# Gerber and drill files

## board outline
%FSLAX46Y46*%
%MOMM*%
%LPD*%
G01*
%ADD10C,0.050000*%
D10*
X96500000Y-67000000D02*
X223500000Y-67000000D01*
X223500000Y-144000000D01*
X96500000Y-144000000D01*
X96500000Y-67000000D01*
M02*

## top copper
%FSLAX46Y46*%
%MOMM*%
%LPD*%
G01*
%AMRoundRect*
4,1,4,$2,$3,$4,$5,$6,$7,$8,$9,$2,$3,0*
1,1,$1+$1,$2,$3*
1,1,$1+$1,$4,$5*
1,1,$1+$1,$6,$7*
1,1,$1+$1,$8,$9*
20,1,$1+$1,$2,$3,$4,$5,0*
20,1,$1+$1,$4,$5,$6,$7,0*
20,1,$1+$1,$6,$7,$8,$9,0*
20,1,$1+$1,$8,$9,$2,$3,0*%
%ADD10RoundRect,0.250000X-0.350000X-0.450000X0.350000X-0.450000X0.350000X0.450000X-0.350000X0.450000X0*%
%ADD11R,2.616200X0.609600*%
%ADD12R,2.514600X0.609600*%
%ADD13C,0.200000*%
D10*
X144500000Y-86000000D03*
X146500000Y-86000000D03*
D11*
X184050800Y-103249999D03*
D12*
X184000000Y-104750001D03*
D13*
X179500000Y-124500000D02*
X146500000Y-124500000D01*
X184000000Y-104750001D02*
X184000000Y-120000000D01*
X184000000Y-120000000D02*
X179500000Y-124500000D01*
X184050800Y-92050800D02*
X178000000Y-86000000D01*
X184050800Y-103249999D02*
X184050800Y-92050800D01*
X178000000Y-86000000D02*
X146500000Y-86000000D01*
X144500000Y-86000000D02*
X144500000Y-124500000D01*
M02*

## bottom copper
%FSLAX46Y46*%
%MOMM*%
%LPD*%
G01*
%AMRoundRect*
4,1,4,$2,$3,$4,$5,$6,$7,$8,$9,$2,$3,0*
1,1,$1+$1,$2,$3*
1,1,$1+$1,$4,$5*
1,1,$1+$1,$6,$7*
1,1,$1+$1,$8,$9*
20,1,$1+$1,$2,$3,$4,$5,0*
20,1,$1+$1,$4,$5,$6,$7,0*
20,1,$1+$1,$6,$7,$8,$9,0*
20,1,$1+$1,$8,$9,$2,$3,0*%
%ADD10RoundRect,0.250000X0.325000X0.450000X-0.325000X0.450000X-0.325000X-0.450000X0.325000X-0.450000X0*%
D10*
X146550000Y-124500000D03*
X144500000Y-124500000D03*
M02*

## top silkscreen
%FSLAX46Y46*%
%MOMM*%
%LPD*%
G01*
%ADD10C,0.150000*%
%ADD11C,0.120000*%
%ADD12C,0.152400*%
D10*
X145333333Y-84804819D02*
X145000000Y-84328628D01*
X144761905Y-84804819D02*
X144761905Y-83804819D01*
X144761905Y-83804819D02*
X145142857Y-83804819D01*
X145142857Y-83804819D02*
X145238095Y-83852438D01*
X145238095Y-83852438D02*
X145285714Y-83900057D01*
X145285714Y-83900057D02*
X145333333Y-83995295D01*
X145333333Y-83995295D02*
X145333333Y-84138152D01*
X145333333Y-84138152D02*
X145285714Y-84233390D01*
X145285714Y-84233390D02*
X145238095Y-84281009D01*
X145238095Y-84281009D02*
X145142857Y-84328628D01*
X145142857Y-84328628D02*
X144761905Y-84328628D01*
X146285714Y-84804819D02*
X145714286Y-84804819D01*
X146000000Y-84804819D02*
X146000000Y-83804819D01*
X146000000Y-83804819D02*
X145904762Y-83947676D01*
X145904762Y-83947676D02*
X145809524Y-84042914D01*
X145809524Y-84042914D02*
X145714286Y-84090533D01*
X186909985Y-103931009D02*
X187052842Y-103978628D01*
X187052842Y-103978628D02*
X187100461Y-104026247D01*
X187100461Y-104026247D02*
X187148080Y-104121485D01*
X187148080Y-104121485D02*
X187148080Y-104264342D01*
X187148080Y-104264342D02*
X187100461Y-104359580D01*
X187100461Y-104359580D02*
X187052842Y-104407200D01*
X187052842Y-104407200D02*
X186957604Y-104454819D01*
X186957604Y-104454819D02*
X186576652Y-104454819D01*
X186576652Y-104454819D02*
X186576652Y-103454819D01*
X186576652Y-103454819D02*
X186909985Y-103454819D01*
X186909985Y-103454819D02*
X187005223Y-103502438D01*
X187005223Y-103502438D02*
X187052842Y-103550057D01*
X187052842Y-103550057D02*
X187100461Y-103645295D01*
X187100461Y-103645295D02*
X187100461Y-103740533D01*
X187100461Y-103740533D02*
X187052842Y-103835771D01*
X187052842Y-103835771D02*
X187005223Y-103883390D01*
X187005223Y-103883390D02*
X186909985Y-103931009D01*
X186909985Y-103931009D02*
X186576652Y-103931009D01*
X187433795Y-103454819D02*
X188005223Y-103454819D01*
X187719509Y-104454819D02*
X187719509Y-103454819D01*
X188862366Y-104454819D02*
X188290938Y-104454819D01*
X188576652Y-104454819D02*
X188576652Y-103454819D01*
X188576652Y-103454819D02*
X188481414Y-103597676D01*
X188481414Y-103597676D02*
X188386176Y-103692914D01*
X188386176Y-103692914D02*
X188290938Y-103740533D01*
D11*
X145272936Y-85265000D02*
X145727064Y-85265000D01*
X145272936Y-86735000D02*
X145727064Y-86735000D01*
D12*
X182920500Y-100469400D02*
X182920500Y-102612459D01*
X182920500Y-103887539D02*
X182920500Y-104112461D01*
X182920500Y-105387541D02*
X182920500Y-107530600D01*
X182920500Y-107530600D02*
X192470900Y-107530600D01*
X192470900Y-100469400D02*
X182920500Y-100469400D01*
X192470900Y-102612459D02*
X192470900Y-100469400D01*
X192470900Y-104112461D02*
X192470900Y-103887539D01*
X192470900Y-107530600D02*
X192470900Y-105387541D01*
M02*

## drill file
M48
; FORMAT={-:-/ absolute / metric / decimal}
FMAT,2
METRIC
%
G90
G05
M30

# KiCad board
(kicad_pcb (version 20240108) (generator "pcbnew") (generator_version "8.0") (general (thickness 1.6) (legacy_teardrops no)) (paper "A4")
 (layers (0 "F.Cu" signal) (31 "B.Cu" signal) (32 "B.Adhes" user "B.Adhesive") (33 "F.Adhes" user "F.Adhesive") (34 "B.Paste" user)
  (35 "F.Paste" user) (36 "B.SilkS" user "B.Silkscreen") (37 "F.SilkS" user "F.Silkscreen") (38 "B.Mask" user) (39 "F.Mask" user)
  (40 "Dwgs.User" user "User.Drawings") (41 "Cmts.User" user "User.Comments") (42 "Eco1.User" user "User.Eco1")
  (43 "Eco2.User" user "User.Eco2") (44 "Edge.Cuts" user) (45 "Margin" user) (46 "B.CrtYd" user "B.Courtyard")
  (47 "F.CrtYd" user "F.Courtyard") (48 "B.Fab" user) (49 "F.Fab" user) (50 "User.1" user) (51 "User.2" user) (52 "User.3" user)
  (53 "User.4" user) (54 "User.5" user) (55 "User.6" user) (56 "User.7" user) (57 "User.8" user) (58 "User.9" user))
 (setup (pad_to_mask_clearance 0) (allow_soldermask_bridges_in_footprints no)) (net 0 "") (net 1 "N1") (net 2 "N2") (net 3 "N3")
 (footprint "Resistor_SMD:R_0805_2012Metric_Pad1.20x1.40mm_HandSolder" (layer "F.Cu") (at 145.5 86)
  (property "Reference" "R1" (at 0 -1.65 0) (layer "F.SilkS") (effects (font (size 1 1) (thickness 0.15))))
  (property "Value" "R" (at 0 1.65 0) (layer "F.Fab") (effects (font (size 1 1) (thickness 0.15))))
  (fp_line (start -0.227064 -0.735) (end 0.227064 -0.735) (stroke (width 0.12) (type solid)) (layer "F.SilkS"))
  (fp_line (start -0.227064 0.735) (end 0.227064 0.735) (stroke (width 0.12) (type solid)) (layer "F.SilkS"))
  (pad "1" smd roundrect (at -1 0) (size 1.2 1.4) (layers "F.Cu" "F.Paste" "F.Mask") (roundrect_rratio 0.208333) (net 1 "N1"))
  (pad "2" smd roundrect (at 1 0) (size 1.2 1.4) (layers "F.Cu" "F.Paste" "F.Mask") (roundrect_rratio 0.208333) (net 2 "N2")))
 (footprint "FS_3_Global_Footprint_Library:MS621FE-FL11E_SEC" (layer "F.Cu") (at 187.6957 104)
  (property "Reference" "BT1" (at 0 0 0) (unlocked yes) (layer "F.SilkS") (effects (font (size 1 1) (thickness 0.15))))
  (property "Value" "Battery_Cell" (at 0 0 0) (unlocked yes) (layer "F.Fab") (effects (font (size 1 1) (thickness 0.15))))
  (fp_line (start -4.7752 -3.5306) (end -4.7752 -1.387541) (stroke (width 0.1524) (type solid)) (layer "F.SilkS"))
  (fp_line (start -4.7752 -0.112461) (end -4.7752 0.112461) (stroke (width 0.1524) (type solid)) (layer "F.SilkS"))
  (fp_line (start -4.7752 1.387541) (end -4.7752 3.5306) (stroke (width 0.1524) (type solid)) (layer "F.SilkS"))
  (fp_line (start -4.7752 3.5306) (end 4.7752 3.5306) (stroke (width 0.1524) (type solid)) (layer "F.SilkS"))
  (fp_line (start 4.7752 -3.5306) (end -4.7752 -3.5306) (stroke (width 0.1524) (type solid)) (layer "F.SilkS"))
  (fp_line (start 4.7752 -1.387541) (end 4.7752 -3.5306) (stroke (width 0.1524) (type solid)) (layer "F.SilkS"))
  (fp_line (start 4.7752 0.112461) (end 4.7752 -0.112461) (stroke (width 0.1524) (type solid)) (layer "F.SilkS"))
  (fp_line (start 4.7752 3.5306) (end 4.7752 1.387541) (stroke (width 0.1524) (type solid)) (layer "F.SilkS"))
  (pad "1" smd rect (at -3.6449 -0.750001) (size 2.6162 0.6096) (layers "F.Cu" "F.Paste" "F.Mask") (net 2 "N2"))
  (pad "2" smd rect (at -3.6957 0.750001) (size 2.5146 0.6096) (layers "F.Cu" "F.Paste" "F.Mask") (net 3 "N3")))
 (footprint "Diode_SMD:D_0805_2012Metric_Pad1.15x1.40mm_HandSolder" (layer "B.Cu") (at 145.525 124.5 180)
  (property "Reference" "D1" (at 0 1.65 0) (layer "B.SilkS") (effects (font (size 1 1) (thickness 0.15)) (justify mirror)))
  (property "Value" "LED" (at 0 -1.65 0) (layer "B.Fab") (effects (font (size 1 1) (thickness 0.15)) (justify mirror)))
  (pad "1" smd roundrect (at -1.025 0 180) (size 1.15 1.4) (layers "B.Cu" "B.Paste" "B.Mask") (roundrect_rratio 0.217391) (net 3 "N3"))
  (pad "2" smd roundrect (at 1.025 0 180) (size 1.15 1.4) (layers "B.Cu" "B.Paste" "B.Mask") (roundrect_rratio 0.217391) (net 1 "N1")))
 (gr_rect (start 96.5 67) (end 223.5 144) (stroke (width 0.05) (type default)) (fill none) (layer "Edge.Cuts"))
 (segment (start 179.5 124.5) (end 146.5 124.5) (width 0.2) (layer "F.Cu") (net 3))
 (segment (start 184 104.750001) (end 184 120) (width 0.2) (layer "F.Cu") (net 3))
 (segment (start 184 120) (end 179.5 124.5) (width 0.2) (layer "F.Cu") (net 3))
 (segment (start 184.0508 92.0508) (end 178 86) (width 0.2) (layer "F.Cu") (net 2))
 (segment (start 184.0508 103.249999) (end 184.0508 92.0508) (width 0.2) (layer "F.Cu") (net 2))
 (segment (start 178 86) (end 146.5 86) (width 0.2) (layer "F.Cu") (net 2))
 (segment (start 144.5 86) (end 144.5 124.5) (width 0.2) (layer "F.Cu") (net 1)))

